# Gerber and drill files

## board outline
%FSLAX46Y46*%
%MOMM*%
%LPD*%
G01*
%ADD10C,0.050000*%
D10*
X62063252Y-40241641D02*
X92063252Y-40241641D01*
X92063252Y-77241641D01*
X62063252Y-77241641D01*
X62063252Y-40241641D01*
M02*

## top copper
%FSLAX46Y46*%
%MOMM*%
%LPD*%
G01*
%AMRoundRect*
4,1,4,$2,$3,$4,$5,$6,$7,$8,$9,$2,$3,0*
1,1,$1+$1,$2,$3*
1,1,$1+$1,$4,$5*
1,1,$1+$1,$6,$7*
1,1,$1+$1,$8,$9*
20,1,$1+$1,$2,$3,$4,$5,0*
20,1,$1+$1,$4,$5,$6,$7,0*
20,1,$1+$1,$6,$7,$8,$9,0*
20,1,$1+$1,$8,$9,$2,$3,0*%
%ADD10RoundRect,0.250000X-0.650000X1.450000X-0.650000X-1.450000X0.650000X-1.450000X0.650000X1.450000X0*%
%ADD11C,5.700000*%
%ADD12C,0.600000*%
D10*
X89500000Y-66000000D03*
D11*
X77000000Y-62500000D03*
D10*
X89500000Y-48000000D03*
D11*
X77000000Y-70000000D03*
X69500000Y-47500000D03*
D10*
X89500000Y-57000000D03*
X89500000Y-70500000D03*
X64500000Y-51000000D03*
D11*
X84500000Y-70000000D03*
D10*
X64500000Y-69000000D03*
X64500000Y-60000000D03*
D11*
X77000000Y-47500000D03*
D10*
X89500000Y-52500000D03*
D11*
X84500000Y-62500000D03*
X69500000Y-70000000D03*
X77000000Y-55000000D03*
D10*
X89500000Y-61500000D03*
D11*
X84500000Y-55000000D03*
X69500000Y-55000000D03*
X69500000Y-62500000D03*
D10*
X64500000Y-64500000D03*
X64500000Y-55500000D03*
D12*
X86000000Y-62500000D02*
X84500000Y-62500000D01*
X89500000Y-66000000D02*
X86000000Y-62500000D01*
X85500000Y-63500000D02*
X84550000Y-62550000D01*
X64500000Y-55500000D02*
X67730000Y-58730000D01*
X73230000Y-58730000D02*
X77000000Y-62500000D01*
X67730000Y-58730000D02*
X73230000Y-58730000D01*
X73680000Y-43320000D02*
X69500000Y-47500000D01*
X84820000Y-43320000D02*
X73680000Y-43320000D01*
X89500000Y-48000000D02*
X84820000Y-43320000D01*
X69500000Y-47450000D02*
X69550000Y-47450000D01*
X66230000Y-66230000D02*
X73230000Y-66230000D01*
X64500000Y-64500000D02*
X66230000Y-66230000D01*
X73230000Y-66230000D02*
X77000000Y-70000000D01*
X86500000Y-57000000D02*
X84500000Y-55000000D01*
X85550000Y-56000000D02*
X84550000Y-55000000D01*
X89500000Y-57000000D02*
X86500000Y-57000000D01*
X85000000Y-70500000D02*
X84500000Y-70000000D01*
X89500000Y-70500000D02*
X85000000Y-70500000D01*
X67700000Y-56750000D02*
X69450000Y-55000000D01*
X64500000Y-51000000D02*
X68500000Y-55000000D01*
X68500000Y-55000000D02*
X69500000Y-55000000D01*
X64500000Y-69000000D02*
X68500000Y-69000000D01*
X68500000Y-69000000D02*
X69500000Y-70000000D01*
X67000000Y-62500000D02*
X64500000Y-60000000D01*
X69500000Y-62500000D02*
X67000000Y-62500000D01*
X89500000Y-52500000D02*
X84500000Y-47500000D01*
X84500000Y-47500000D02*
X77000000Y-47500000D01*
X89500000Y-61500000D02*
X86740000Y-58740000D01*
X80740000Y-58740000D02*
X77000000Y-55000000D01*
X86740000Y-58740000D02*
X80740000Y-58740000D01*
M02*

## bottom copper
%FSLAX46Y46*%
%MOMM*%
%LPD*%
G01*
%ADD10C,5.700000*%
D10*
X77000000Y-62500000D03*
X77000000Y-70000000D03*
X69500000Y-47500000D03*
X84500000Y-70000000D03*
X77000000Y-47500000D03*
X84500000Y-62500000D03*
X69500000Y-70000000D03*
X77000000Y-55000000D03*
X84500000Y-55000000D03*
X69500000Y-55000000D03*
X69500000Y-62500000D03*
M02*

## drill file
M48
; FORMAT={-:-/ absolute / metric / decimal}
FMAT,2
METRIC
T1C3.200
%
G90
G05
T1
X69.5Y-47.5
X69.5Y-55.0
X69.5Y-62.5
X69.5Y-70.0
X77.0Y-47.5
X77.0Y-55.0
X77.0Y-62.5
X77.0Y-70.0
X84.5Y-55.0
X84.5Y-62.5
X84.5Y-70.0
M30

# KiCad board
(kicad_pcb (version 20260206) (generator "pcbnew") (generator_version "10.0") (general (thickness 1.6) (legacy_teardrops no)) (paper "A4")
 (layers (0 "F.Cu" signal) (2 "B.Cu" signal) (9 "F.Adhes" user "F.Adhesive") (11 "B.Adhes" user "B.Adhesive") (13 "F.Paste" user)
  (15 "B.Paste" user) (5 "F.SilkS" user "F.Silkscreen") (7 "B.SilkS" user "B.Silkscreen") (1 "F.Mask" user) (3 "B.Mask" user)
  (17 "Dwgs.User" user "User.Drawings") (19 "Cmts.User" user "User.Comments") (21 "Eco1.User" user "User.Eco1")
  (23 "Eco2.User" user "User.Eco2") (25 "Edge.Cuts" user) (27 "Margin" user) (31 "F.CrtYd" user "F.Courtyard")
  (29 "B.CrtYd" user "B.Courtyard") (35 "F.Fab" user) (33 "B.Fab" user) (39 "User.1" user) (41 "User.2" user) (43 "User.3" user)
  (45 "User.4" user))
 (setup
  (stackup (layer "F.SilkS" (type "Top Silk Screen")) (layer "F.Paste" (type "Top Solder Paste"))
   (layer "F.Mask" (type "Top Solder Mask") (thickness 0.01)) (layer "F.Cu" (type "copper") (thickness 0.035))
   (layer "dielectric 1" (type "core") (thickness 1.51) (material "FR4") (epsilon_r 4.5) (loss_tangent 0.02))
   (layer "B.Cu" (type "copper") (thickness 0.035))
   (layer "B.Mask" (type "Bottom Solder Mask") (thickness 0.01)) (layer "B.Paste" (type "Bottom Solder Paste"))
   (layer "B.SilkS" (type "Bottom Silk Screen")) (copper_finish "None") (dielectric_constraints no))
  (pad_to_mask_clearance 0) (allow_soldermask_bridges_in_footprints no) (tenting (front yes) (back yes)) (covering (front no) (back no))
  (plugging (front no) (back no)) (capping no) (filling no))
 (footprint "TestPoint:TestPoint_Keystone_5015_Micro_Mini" (layer "F.Cu") (at 89.5 66 -90)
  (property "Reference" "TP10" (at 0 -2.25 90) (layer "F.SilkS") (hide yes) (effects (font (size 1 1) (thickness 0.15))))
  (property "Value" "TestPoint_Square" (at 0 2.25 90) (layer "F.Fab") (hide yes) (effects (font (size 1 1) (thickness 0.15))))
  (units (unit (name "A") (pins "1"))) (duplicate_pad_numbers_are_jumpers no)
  (pad "1" smd roundrect (at 0 0 270) (size 3.4 1.8) (layers "F.Cu" "F.Mask" "F.Paste") (roundrect_rratio 0.1388888889)
   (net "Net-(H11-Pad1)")))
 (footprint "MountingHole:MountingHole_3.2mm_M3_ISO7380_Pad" (layer "F.Cu") (at 77 62.5)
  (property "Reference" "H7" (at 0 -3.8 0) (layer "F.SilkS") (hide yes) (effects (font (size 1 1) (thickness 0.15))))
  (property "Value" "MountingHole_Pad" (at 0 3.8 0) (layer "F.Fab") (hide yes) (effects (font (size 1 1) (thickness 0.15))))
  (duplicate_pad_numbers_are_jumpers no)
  (pad "1" thru_hole circle (at 0 0) (size 5.7 5.7) (drill 3.2) (layers "*.Cu" "*.Mask") (remove_unused_layers no) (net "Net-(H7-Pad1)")
   (zone_connect 2)))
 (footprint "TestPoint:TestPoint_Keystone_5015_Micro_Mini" (layer "F.Cu") (at 89.5 48 -90)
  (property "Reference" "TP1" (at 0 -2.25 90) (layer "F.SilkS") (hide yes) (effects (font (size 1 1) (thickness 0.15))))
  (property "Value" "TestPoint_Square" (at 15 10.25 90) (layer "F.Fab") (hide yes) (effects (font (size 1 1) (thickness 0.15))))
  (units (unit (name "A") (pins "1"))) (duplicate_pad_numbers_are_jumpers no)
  (pad "1" smd roundrect (at 0 0 270) (size 3.4 1.8) (layers "F.Cu" "F.Mask" "F.Paste") (roundrect_rratio 0.1388888889)
   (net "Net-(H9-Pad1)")))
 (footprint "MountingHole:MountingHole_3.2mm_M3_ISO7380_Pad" (layer "F.Cu") (at 77 70)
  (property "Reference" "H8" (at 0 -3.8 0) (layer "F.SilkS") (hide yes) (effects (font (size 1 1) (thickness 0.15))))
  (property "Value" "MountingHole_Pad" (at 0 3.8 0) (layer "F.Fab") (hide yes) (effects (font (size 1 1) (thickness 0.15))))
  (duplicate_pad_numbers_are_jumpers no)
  (pad "1" thru_hole circle (at 0 0) (size 5.7 5.7) (drill 3.2) (layers "*.Cu" "*.Mask") (remove_unused_layers no) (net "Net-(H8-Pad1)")
   (zone_connect 2)))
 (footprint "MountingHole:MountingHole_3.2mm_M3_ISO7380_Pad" (layer "F.Cu") (at 69.5 47.5)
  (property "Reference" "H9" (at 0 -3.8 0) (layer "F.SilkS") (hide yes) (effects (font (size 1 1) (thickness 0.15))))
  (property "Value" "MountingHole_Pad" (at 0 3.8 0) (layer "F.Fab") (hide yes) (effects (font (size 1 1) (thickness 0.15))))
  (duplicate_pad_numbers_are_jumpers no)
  (pad "1" thru_hole circle (at 0 0) (size 5.7 5.7) (drill 3.2) (layers "*.Cu" "*.Mask") (remove_unused_layers no) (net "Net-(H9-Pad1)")
   (zone_connect 2)))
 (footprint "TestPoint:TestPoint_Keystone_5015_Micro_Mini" (layer "F.Cu") (at 89.5 57 -90)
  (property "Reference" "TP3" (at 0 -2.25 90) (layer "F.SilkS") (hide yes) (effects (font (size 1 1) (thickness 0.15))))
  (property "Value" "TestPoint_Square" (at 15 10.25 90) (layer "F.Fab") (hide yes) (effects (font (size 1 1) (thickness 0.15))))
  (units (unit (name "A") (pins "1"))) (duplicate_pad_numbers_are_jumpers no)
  (pad "1" smd roundrect (at 0 0 270) (size 3.4 1.8) (layers "F.Cu" "F.Mask" "F.Paste") (roundrect_rratio 0.1388888889)
   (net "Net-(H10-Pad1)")))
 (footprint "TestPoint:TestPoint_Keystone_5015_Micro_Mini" (layer "F.Cu") (at 89.5 70.5 -90)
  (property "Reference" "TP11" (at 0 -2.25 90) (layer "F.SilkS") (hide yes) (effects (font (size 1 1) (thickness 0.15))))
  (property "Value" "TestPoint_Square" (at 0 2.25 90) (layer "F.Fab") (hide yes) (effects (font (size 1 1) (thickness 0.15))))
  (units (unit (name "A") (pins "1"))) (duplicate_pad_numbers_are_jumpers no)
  (pad "1" smd roundrect (at 0 0 270) (size 3.4 1.8) (layers "F.Cu" "F.Mask" "F.Paste") (roundrect_rratio 0.1388888889)
   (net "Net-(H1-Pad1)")))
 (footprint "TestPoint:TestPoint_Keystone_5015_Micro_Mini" (layer "F.Cu") (at 64.5 51 -90)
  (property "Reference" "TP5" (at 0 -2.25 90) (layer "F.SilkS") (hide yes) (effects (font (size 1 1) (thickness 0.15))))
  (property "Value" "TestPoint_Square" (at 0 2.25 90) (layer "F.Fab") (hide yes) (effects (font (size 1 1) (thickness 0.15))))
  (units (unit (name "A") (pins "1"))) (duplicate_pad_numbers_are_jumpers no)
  (pad "1" smd roundrect (at 0 0 270) (size 3.4 1.8) (layers "F.Cu" "F.Mask" "F.Paste") (roundrect_rratio 0.1388888889)
   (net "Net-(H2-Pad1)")))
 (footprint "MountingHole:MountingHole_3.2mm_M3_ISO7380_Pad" (layer "F.Cu") (at 84.5 70)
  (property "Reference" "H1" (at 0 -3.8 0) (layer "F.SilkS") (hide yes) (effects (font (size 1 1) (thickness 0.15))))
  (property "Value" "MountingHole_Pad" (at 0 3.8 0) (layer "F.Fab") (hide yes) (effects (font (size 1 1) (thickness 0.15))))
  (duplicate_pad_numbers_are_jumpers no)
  (pad "1" thru_hole circle (at 0 0) (size 5.7 5.7) (drill 3.2) (layers "*.Cu" "*.Mask") (remove_unused_layers no) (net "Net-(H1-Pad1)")
   (zone_connect 2)))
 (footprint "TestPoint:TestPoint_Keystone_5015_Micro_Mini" (layer "F.Cu") (at 64.5 69 -90)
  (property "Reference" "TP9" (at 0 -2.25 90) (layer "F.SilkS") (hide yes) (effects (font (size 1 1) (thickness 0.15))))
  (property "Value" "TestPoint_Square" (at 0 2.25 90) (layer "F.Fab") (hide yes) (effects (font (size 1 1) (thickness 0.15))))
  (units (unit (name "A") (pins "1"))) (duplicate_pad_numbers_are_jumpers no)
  (pad "1" smd roundrect (at 0 0 270) (size 3.4 1.8) (layers "F.Cu" "F.Mask" "F.Paste") (roundrect_rratio 0.1388888889)
   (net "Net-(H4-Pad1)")))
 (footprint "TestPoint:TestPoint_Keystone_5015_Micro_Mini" (layer "F.Cu") (at 64.5 60 -90)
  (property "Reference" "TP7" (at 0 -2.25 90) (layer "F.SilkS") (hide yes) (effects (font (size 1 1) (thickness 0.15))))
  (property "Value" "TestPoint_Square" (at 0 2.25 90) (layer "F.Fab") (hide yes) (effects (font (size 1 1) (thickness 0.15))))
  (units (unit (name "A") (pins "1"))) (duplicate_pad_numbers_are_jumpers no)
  (pad "1" smd roundrect (at 0 0 270) (size 3.4 1.8) (layers "F.Cu" "F.Mask" "F.Paste") (roundrect_rratio 0.1388888889)
   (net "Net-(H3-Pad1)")))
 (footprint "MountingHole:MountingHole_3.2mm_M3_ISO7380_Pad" (layer "F.Cu") (at 77 47.5)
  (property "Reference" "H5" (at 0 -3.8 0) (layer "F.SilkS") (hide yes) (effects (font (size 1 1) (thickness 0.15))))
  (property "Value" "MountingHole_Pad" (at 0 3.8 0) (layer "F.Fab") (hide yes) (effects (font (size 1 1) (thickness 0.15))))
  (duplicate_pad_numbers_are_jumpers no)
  (pad "1" thru_hole circle (at 0 0) (size 5.7 5.7) (drill 3.2) (layers "*.Cu" "*.Mask") (remove_unused_layers no) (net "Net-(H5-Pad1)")
   (zone_connect 2)))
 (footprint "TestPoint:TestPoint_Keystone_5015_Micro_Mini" (layer "F.Cu") (at 89.5 52.5 -90)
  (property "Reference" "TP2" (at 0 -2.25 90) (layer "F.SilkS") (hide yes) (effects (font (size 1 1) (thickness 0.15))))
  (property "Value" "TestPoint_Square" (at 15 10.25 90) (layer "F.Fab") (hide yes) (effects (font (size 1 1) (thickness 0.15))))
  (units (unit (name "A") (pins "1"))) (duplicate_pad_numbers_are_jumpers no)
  (pad "1" smd roundrect (at 0 0 270) (size 3.4 1.8) (layers "F.Cu" "F.Mask" "F.Paste") (roundrect_rratio 0.1388888889)
   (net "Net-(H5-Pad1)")))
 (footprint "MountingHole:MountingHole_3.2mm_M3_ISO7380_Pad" (layer "F.Cu") (at 84.5 62.5)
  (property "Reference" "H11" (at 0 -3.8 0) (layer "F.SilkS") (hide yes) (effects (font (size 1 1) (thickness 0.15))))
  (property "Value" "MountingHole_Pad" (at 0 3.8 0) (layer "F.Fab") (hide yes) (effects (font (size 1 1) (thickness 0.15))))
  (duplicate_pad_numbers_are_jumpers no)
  (pad "1" thru_hole circle (at 0 0) (size 5.7 5.7) (drill 3.2) (layers "*.Cu" "*.Mask") (remove_unused_layers no) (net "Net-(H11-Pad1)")
   (zone_connect 2)))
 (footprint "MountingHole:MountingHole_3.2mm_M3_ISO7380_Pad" (layer "F.Cu") (at 69.5 70)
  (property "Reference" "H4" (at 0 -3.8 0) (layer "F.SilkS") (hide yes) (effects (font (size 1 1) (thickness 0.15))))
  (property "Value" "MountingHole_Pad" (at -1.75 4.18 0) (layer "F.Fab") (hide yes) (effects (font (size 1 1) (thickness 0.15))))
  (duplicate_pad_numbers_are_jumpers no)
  (pad "1" thru_hole circle (at 0 0) (size 5.7 5.7) (drill 3.2) (layers "*.Cu" "*.Mask") (remove_unused_layers no) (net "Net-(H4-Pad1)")
   (zone_connect 2)))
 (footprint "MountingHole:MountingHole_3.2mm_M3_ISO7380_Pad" (layer "F.Cu") (at 77 55)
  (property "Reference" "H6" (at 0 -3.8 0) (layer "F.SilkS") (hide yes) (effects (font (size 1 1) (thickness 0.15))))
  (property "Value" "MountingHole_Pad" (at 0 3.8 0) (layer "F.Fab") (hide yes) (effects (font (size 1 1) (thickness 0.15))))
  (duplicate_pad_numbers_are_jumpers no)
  (pad "1" thru_hole circle (at 0 0) (size 5.7 5.7) (drill 3.2) (layers "*.Cu" "*.Mask") (remove_unused_layers no) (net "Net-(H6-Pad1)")
   (zone_connect 2)))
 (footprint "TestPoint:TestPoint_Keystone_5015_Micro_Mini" (layer "F.Cu") (at 89.5 61.5 -90)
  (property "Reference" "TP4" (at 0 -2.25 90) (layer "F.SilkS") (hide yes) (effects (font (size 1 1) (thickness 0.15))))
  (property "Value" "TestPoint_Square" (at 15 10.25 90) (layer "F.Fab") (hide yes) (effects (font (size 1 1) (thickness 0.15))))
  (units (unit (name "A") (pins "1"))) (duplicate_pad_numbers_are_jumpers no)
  (pad "1" smd roundrect (at 0 0 270) (size 3.4 1.8) (layers "F.Cu" "F.Mask" "F.Paste") (roundrect_rratio 0.1388888889)
   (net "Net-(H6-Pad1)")))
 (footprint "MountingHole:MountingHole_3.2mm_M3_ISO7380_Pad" (layer "F.Cu") (at 84.5 55)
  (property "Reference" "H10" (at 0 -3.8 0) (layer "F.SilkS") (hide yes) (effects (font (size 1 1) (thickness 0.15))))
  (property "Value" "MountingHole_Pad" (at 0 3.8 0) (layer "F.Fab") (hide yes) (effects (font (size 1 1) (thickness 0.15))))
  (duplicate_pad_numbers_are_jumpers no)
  (pad "1" thru_hole circle (at 0 0) (size 5.7 5.7) (drill 3.2) (layers "*.Cu" "*.Mask") (remove_unused_layers no) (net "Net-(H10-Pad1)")
   (zone_connect 2)))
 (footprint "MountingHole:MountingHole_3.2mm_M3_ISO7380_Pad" (layer "F.Cu") (at 69.5 55)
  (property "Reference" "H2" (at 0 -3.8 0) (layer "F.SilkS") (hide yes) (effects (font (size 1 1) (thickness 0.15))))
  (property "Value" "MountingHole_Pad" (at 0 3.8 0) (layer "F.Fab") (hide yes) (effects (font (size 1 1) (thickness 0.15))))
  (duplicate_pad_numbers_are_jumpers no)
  (pad "1" thru_hole circle (at 0 0) (size 5.7 5.7) (drill 3.2) (layers "*.Cu" "*.Mask") (remove_unused_layers no) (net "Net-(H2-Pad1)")
   (zone_connect 2)))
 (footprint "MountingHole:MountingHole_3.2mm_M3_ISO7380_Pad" (layer "F.Cu") (at 69.5 62.5)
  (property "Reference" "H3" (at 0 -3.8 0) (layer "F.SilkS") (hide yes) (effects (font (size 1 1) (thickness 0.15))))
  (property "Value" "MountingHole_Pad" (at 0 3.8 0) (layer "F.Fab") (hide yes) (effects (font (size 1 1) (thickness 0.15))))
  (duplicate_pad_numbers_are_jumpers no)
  (pad "1" thru_hole circle (at 0 0) (size 5.7 5.7) (drill 3.2) (layers "*.Cu" "*.Mask") (remove_unused_layers no) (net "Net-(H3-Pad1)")
   (zone_connect 2)))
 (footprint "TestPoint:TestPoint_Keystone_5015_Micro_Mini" (layer "F.Cu") (at 64.5 64.5 -90)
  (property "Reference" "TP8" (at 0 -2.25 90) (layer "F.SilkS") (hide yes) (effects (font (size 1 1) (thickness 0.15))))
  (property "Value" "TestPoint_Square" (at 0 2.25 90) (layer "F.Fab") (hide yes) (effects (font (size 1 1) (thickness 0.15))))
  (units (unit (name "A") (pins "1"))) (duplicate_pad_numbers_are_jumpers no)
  (pad "1" smd roundrect (at 0 0 270) (size 3.4 1.8) (layers "F.Cu" "F.Mask" "F.Paste") (roundrect_rratio 0.1388888889)
   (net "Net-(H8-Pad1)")))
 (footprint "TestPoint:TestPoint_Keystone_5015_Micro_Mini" (layer "F.Cu") (at 64.5 55.5 -90)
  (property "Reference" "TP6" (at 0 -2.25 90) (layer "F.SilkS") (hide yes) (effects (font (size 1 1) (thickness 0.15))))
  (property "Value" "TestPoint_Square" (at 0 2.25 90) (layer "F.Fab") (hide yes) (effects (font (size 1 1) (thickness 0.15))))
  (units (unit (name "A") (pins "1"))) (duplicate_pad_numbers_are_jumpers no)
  (pad "1" smd roundrect (at 0 0 270) (size 3.4 1.8) (layers "F.Cu" "F.Mask" "F.Paste") (roundrect_rratio 0.1388888889)
   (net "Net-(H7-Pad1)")))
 (gr_rect (start 62.063252 40.241641) (end 92.063252 77.241641) (stroke (width 0.05) (type default)) (fill no) (layer "Edge.Cuts"))
 (segment (start 86 62.5) (end 84.5 62.5) (width 0.6) (layer "F.Cu") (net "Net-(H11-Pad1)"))
 (segment (start 89.5 66) (end 86 62.5) (width 0.6) (layer "F.Cu") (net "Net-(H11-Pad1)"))
 (segment (start 85.5 63.5) (end 84.55 62.55) (width 0.6) (layer "F.Cu") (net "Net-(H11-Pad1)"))
 (segment (start 64.5 55.5) (end 67.73 58.73) (width 0.6) (layer "F.Cu") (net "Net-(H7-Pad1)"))
 (segment (start 73.23 58.73) (end 77 62.5) (width 0.6) (layer "F.Cu") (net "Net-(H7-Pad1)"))
 (segment (start 67.73 58.73) (end 73.23 58.73) (width 0.6) (layer "F.Cu") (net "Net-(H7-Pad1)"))
 (segment (start 73.68 43.32) (end 69.5 47.5) (width 0.6) (layer "F.Cu") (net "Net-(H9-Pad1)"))
 (segment (start 84.82 43.32) (end 73.68 43.32) (width 0.6) (layer "F.Cu") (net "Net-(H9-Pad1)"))
 (segment (start 89.5 48) (end 84.82 43.32) (width 0.6) (layer "F.Cu") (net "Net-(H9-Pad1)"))
 (segment (start 69.5 47.45) (end 69.55 47.45) (width 0.6) (layer "F.Cu") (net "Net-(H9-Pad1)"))
 (segment (start 66.23 66.23) (end 73.23 66.23) (width 0.6) (layer "F.Cu") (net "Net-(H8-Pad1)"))
 (segment (start 64.5 64.5) (end 66.23 66.23) (width 0.6) (layer "F.Cu") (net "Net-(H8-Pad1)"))
 (segment (start 73.23 66.23) (end 77 70) (width 0.6) (layer "F.Cu") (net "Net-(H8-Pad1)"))
 (segment (start 86.5 57) (end 84.5 55) (width 0.6) (layer "F.Cu") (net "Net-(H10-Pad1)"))
 (segment (start 85.55 56) (end 84.55 55) (width 0.6) (layer "F.Cu") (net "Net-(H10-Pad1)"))
 (segment (start 89.5 57) (end 86.5 57) (width 0.6) (layer "F.Cu") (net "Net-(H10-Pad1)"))
 (segment (start 85 70.5) (end 84.5 70) (width 0.6) (layer "F.Cu") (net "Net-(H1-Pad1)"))
 (segment (start 89.5 70.5) (end 85 70.5) (width 0.6) (layer "F.Cu") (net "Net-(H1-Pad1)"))
 (segment (start 67.7 56.75) (end 69.45 55) (width 0.6) (layer "F.Cu") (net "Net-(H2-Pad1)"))
 (segment (start 64.5 51) (end 68.5 55) (width 0.6) (layer "F.Cu") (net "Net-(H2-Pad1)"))
 (segment (start 68.5 55) (end 69.5 55) (width 0.6) (layer "F.Cu") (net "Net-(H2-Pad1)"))
 (segment (start 64.5 69) (end 68.5 69) (width 0.6) (layer "F.Cu") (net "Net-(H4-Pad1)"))
 (segment (start 68.5 69) (end 69.5 70) (width 0.6) (layer "F.Cu") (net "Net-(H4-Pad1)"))
 (segment (start 67 62.5) (end 64.5 60) (width 0.6) (layer "F.Cu") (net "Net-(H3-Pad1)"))
 (segment (start 69.5 62.5) (end 67 62.5) (width 0.6) (layer "F.Cu") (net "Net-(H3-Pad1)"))
 (segment (start 89.5 52.5) (end 84.5 47.5) (width 0.6) (layer "F.Cu") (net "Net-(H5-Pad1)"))
 (segment (start 84.5 47.5) (end 77 47.5) (width 0.6) (layer "F.Cu") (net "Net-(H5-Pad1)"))
 (segment (start 89.5 61.5) (end 86.74 58.74) (width 0.6) (layer "F.Cu") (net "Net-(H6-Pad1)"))
 (segment (start 80.74 58.74) (end 77 55) (width 0.6) (layer "F.Cu") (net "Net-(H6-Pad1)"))
 (segment (start 86.74 58.74) (end 80.74 58.74) (width 0.6) (layer "F.Cu") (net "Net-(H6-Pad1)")))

